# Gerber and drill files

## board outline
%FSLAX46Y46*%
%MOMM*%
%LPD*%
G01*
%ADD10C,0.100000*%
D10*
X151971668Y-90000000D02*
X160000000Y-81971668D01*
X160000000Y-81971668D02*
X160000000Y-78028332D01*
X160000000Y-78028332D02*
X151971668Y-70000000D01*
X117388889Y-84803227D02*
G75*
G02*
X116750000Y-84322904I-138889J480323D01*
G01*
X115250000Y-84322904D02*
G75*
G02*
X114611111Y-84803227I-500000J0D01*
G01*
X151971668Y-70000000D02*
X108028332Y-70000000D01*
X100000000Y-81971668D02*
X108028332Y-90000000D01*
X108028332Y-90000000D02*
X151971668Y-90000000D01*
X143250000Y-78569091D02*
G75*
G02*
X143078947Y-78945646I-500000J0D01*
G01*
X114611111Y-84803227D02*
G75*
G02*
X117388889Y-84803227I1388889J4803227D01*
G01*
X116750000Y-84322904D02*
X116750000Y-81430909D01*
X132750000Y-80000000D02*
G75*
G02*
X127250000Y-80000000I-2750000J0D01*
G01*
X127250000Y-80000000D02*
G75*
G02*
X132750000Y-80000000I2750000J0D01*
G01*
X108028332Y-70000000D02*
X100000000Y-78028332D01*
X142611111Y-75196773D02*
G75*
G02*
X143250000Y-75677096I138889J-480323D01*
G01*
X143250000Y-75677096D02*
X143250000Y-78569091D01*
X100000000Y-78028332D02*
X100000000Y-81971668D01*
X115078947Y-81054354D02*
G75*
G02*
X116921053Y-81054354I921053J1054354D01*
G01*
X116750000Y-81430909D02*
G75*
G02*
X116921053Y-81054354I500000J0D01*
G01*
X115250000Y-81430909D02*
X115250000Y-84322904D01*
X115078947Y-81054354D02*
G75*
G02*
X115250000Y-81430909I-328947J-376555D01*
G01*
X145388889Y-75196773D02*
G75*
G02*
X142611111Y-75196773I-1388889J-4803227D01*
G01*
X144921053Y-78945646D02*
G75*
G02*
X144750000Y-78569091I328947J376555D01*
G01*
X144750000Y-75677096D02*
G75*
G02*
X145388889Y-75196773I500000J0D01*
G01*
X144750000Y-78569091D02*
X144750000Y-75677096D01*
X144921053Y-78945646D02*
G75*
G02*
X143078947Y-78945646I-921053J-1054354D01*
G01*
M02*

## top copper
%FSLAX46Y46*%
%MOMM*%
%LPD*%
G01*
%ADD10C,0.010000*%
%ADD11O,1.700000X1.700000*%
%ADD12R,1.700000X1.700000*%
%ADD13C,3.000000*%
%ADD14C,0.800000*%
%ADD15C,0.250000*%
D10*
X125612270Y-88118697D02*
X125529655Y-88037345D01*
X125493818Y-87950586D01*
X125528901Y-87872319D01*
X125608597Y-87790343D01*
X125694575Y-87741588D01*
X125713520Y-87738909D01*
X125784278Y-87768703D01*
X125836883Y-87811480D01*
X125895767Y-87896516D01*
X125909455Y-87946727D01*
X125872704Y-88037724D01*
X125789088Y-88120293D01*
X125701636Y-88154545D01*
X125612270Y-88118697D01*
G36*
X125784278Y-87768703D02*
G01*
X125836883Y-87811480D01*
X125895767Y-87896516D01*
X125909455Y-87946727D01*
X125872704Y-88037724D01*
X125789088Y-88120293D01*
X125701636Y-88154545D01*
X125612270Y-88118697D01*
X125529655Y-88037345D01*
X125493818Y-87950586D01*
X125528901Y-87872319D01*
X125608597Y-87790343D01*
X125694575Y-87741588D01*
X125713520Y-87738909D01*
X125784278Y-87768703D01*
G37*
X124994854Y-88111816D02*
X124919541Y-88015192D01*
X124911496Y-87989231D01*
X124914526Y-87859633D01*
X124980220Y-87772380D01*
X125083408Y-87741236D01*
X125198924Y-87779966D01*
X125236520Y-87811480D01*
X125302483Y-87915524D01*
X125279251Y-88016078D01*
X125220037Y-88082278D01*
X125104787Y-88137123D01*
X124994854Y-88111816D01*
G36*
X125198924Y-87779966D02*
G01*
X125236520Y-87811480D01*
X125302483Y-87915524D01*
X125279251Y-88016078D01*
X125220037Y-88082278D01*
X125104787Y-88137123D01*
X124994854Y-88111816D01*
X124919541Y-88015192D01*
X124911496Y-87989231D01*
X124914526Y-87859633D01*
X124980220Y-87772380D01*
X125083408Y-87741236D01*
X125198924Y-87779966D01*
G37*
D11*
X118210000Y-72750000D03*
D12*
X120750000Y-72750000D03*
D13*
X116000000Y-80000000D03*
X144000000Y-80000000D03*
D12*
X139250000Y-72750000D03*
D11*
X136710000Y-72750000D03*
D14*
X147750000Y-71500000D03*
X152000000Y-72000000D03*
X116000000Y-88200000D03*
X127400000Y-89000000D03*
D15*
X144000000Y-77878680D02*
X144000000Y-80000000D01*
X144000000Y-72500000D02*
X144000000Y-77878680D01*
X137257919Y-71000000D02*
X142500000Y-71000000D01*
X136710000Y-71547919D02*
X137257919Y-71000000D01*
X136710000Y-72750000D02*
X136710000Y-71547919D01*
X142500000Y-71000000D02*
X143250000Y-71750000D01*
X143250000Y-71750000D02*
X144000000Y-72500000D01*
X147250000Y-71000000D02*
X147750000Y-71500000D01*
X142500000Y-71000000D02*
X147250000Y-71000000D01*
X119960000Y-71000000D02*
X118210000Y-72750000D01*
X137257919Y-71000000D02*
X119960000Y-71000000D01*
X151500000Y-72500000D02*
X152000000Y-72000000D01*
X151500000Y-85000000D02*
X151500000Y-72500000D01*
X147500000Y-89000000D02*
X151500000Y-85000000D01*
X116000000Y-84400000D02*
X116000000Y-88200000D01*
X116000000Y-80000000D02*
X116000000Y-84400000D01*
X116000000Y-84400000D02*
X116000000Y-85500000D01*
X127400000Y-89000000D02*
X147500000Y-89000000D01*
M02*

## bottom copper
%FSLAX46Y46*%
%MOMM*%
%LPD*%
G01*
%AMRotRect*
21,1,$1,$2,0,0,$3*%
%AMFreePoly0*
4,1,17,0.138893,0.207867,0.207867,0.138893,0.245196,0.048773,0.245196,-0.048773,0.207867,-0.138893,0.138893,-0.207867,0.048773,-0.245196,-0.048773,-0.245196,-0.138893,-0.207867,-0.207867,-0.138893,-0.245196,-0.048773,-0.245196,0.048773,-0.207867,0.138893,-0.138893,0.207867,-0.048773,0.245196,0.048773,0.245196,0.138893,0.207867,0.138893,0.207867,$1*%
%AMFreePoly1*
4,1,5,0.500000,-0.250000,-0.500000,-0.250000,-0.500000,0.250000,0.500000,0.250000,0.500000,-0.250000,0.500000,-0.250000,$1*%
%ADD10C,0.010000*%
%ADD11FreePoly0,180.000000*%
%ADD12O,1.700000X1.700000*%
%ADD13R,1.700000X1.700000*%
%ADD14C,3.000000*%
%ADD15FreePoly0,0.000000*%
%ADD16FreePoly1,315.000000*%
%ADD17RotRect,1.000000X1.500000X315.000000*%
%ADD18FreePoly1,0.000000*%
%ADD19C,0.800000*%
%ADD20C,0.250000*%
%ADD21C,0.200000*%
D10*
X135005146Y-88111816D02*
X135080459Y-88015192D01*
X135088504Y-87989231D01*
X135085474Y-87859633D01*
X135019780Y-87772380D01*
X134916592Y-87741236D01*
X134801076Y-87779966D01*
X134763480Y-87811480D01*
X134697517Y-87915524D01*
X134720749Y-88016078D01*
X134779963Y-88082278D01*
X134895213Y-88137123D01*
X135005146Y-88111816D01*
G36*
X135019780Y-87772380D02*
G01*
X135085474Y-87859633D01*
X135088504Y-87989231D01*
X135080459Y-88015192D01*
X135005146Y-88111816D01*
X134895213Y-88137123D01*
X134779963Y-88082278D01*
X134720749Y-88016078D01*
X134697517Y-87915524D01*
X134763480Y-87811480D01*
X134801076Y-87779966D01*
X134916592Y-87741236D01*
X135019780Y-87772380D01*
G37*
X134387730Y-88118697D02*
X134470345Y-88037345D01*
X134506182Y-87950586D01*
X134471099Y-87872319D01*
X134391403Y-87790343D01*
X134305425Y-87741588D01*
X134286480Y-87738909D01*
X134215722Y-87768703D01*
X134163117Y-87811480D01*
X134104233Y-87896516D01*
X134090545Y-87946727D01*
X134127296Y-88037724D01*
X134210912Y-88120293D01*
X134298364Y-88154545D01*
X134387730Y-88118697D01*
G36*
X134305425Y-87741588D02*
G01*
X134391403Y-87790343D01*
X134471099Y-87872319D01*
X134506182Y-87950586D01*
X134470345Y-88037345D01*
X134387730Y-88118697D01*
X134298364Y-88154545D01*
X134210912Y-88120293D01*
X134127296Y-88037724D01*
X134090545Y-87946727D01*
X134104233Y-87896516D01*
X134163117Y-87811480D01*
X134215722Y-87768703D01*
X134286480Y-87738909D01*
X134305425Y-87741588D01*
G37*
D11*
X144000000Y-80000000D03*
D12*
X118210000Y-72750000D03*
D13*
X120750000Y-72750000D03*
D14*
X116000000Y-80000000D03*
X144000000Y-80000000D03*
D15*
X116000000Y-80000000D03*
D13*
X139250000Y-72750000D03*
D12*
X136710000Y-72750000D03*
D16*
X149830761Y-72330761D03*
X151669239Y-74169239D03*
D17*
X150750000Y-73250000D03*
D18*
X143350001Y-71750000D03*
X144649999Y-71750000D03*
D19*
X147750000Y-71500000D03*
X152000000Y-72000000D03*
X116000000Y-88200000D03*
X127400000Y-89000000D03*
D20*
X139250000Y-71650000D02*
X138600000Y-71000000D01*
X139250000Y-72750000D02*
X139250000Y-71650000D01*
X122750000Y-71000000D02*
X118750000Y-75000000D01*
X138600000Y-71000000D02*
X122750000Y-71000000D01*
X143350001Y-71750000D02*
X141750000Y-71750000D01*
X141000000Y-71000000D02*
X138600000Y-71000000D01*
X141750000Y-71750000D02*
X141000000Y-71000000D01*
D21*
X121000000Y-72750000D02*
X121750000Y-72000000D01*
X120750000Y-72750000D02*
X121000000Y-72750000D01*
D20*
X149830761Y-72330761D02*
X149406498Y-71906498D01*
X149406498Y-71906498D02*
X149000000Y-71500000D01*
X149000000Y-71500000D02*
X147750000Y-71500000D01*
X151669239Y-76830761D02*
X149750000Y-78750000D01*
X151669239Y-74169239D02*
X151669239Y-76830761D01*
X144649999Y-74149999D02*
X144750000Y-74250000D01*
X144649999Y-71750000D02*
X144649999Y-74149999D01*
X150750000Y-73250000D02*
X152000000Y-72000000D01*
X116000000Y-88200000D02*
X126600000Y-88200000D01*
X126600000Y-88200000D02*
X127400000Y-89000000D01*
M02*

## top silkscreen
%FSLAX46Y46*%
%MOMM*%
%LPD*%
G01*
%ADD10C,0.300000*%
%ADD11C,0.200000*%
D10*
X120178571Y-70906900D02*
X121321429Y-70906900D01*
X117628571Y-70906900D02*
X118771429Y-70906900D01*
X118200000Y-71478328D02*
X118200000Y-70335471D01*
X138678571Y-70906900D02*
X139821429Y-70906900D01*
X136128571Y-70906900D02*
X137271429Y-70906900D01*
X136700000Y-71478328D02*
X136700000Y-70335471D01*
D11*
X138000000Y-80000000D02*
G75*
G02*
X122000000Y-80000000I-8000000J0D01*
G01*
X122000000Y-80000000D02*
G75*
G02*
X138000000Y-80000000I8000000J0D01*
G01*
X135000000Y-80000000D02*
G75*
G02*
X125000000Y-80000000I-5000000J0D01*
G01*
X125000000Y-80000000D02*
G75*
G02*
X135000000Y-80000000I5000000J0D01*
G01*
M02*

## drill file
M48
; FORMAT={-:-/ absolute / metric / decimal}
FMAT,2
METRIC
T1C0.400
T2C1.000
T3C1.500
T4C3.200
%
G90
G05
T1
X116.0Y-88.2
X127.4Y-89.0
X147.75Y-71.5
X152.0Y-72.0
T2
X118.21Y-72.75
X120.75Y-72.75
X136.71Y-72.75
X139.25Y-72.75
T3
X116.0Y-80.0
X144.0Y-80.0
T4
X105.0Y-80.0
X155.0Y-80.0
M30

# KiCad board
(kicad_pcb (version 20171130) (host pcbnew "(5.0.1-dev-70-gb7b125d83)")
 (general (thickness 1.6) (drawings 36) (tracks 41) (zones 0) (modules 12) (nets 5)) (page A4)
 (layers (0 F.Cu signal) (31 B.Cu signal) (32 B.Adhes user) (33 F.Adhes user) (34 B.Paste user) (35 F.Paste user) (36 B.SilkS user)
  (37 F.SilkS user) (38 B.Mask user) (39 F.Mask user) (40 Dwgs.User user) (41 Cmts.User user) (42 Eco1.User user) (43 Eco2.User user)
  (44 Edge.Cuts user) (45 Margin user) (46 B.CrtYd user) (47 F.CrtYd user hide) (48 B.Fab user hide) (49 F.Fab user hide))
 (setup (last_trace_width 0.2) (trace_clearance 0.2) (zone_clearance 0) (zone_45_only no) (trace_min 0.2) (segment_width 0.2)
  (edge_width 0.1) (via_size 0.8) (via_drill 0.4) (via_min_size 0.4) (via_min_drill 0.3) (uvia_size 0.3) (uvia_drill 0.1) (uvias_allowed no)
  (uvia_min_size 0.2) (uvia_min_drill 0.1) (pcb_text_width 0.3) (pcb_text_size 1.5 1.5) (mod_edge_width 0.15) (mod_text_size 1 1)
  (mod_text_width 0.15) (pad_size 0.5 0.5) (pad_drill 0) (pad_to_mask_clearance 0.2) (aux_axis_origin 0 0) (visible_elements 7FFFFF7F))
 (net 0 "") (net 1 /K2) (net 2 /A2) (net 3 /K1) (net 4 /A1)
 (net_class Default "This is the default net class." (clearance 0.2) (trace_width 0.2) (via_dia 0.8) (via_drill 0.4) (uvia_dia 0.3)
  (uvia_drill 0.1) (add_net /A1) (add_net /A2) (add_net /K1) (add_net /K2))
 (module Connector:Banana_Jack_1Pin (layer F.Cu) (at 75.6 77.6 180)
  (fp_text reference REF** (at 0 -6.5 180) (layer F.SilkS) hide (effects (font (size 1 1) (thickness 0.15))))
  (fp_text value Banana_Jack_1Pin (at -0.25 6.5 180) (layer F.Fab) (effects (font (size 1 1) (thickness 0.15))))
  (pad e smd custom (at -68.4 -2.4 180) (size 0.5 0.5) (layers B.Cu B.Paste B.Mask) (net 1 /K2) (zone_connect 0)
   (options (clearance outline) (anchor circle)) (primitives)))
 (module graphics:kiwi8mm (layer F.Cu) (at 123 87 180)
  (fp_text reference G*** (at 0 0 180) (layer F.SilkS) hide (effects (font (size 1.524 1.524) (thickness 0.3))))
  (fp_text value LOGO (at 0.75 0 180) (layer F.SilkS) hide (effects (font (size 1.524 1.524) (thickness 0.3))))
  (fp_poly
   (pts (xy -2.61227 -1.118697) (xy -2.529655 -1.037345) (xy -2.493818 -0.950586) (xy -2.528901 -0.872319) (xy -2.608597 -0.790343)
    (xy -2.694575 -0.741588) (xy -2.71352 -0.738909) (xy -2.784278 -0.768703) (xy -2.836883 -0.81148) (xy -2.895767 -0.896516)
    (xy -2.909455 -0.946727) (xy -2.872704 -1.037724) (xy -2.789088 -1.120293) (xy -2.701636 -1.154545) (xy -2.61227 -1.118697))
   (layer F.Cu) (width 0.01))
  (fp_poly
   (pts (xy -1.994854 -1.111816) (xy -1.919541 -1.015192) (xy -1.911496 -0.989231) (xy -1.914526 -0.859633) (xy -1.98022 -0.77238)
    (xy -2.083408 -0.741236) (xy -2.198924 -0.779966) (xy -2.23652 -0.81148) (xy -2.302483 -0.915524) (xy -2.279251 -1.016078)
    (xy -2.220037 -1.082278) (xy -2.104787 -1.137123) (xy -1.994854 -1.111816))
   (layer F.Cu) (width 0.01)))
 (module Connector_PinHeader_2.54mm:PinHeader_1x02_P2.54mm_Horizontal (layer B.Cu) (at 120.75 72.75 90)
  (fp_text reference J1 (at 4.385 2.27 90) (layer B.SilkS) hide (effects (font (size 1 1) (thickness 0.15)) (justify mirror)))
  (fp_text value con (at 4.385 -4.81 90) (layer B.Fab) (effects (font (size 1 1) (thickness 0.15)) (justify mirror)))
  (pad 2 thru_hole oval (at 0 -2.54 90) (size 1.7 1.7) (drill 1) (layers *.Cu *.Mask) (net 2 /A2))
  (pad 1 thru_hole rect (at 0 0 90) (size 1.7 1.7) (drill 1) (layers *.Cu *.Mask) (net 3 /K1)))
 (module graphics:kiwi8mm (layer B.Cu) (at 137 87)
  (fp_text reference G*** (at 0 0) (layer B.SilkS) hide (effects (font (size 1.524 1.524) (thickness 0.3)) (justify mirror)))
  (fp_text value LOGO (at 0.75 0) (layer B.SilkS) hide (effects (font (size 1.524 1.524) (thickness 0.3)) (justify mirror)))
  (fp_poly
   (pts (xy -1.994854 1.111816) (xy -1.919541 1.015192) (xy -1.911496 0.989231) (xy -1.914526 0.859633) (xy -1.98022 0.77238)
    (xy -2.083408 0.741236) (xy -2.198924 0.779966) (xy -2.23652 0.81148) (xy -2.302483 0.915524) (xy -2.279251 1.016078)
    (xy -2.220037 1.082278) (xy -2.104787 1.137123) (xy -1.994854 1.111816))
   (layer B.Cu) (width 0.01))
  (fp_poly
   (pts (xy -2.61227 1.118697) (xy -2.529655 1.037345) (xy -2.493818 0.950586) (xy -2.528901 0.872319) (xy -2.608597 0.790343)
    (xy -2.694575 0.741588) (xy -2.71352 0.738909) (xy -2.784278 0.768703) (xy -2.836883 0.81148) (xy -2.895767 0.896516)
    (xy -2.909455 0.946727) (xy -2.872704 1.037724) (xy -2.789088 1.120293) (xy -2.701636 1.154545) (xy -2.61227 1.118697))
   (layer B.Cu) (width 0.01)))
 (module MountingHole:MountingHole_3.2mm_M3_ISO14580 (layer F.Cu) (at 105 80)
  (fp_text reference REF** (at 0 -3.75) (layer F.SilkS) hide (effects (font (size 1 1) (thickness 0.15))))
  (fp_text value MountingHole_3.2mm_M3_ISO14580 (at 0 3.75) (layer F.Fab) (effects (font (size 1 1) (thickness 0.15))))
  (pad 1 np_thru_hole circle (at 0 0) (size 3.2 3.2) (drill 3.2) (layers *.Cu *.Mask)))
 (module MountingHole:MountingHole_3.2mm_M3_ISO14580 (layer F.Cu) (at 155 80)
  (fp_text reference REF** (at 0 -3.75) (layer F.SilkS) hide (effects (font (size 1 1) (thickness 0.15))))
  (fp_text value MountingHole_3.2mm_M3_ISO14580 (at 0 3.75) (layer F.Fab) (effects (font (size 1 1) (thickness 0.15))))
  (pad 1 np_thru_hole circle (at 0 0) (size 3.2 3.2) (drill 3.2) (layers *.Cu *.Mask)))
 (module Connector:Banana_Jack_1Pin (layer F.Cu) (at 175.6 64.6)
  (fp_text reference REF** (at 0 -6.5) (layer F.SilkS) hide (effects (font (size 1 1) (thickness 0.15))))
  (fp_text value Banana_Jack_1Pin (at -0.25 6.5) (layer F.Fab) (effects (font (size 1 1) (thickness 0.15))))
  (pad 1 thru_hole circle (at -59.6 15.4) (size 3 3) (drill 1.5) (layers *.Cu *.Mask) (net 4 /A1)))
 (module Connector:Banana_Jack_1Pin (layer F.Cu) (at 203.6 64.6)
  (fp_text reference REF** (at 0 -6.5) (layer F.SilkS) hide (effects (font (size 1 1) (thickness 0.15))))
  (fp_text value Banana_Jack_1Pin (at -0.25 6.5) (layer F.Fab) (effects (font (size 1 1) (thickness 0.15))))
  (pad 1 thru_hole circle (at -59.6 15.4) (size 3 3) (drill 1.5) (layers *.Cu *.Mask) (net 2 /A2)))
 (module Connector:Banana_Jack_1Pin (layer F.Cu) (at 184.4 82.4)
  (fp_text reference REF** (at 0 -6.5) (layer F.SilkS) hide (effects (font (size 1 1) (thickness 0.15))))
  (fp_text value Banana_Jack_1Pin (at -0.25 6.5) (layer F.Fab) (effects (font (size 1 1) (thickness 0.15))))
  (pad e smd custom (at -68.4 -2.4) (size 0.5 0.5) (layers B.Cu B.Paste B.Mask) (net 3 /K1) (zone_connect 0)
   (options (clearance outline) (anchor circle)) (primitives)))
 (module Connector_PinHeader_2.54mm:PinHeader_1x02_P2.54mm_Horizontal (layer B.Cu) (at 139.25 72.75 90)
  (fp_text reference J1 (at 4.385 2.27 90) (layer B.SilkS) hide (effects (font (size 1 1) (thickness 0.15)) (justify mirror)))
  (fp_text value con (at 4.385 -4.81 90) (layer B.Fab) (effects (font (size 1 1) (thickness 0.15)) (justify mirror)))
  (pad 1 thru_hole rect (at 0 0 90) (size 1.7 1.7) (drill 1) (layers *.Cu *.Mask) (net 3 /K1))
  (pad 2 thru_hole oval (at 0 -2.54 90) (size 1.7 1.7) (drill 1) (layers *.Cu *.Mask) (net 2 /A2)))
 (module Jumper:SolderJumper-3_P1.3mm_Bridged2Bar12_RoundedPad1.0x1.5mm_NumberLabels (layer B.Cu) (at 150.75 73.25 315)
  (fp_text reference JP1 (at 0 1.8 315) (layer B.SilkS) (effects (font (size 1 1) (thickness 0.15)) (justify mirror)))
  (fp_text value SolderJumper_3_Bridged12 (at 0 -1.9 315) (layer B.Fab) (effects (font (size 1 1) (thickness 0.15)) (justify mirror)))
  (pad 1 smd custom (at -1.3 0 315) (size 1 0.5) (layers B.Cu B.Mask) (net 2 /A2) (zone_connect 0)
   (options (clearance outline) (anchor rect)) (primitives))
  (pad 3 smd custom (at 1.3 0 315) (size 1 0.5) (layers B.Cu B.Mask) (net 1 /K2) (zone_connect 0)
   (options (clearance outline) (anchor rect)) (primitives))
  (pad 2 smd rect (at 0 0 315) (size 1 1.5) (layers B.Cu B.Mask) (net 4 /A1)))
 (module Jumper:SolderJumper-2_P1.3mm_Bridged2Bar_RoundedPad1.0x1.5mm (layer B.Cu) (at 144 71.75)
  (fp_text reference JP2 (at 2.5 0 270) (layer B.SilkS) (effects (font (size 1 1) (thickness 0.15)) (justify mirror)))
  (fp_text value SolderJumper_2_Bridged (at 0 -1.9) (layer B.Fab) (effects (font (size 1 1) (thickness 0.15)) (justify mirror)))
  (pad 1 smd custom (at -0.649999 0) (size 1 0.5) (layers B.Cu B.Mask) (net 3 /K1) (zone_connect 0)
   (options (clearance outline) (anchor rect)) (primitives))
  (pad 2 smd custom (at 0.649999 0) (size 1 0.5) (layers B.Cu B.Mask) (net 1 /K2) (zone_connect 0)
   (options (clearance outline) (anchor rect)) (primitives)))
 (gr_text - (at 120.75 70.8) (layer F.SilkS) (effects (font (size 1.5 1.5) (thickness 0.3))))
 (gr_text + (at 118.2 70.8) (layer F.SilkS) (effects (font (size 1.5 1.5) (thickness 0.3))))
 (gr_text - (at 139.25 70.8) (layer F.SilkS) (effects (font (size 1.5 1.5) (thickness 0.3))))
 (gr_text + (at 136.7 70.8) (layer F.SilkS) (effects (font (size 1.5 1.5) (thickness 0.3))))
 (gr_line (start 151.971668 90) (end 160 81.971668) (layer Edge.Cuts) (width 0.1))
 (gr_line (start 160 81.971668) (end 160 78.028332) (layer Edge.Cuts) (width 0.1))
 (gr_line (start 160 78.028332) (end 151.971668 70) (layer Edge.Cuts) (width 0.1))
 (gr_circle (center 130 80) (end 138 80) (layer F.SilkS) (width 0.2))
 (gr_circle (center 130 80) (end 125 80) (layer F.SilkS) (width 0.2))
 (gr_arc (start 117.25 84.322904) (end 116.75 84.322904) (angle -106.1276202) (layer Edge.Cuts) (width 0.1))
 (gr_arc (start 114.75 84.322904) (end 114.611111 84.803227) (angle -106.1276202) (layer Edge.Cuts) (width 0.1))
 (gr_line (start 151.971668 70) (end 108.028332 70) (layer Edge.Cuts) (width 0.1))
 (gr_line (start 100 81.971668) (end 108.028332 90) (layer Edge.Cuts) (width 0.1))
 (gr_line (start 108.028332 90) (end 151.971668 90) (layer Edge.Cuts) (width 0.1))
 (gr_arc (start 142.75 78.569091) (end 143.078947 78.945646) (angle -48.86048959) (layer Edge.Cuts) (width 0.1))
 (gr_arc (start 116 80) (end 117.388889 84.803227) (angle -327.7447596) (layer Edge.Cuts) (width 0.1))
 (gr_line (start 116.75 84.322904) (end 116.75 81.430909) (layer Edge.Cuts) (width 0.1))
 (gr_circle (center 130 80) (end 132.75 80) (layer Edge.Cuts) (width 0.1))
 (gr_line (start 108.028332 70) (end 100 78.028332) (layer Edge.Cuts) (width 0.1))
 (gr_arc (start 142.75 75.677096) (end 143.25 75.677096) (angle -106.1276202) (layer Edge.Cuts) (width 0.1))
 (gr_line (start 143.25 75.677096) (end 143.25 78.569091) (layer Edge.Cuts) (width 0.1))
 (gr_line (start 100 78.028332) (end 100 81.971668) (layer Edge.Cuts) (width 0.1))
 (gr_arc (start 116 80) (end 116.921053 81.054354) (angle -277.7209792) (layer Edge.Cuts) (width 0.1))
 (gr_arc (start 117.25 81.430909) (end 116.921053 81.054354) (angle -48.86048959) (layer Edge.Cuts) (width 0.1))
 (gr_line (start 115.25 81.430909) (end 115.25 84.322904) (layer Edge.Cuts) (width 0.1))
 (gr_arc (start 114.75 81.430909) (end 115.25 81.430909) (angle -48.86048959) (layer Edge.Cuts) (width 0.1))
 (gr_arc (start 144 80) (end 142.611111 75.196773) (angle -327.7447596) (layer Edge.Cuts) (width 0.1))
 (gr_arc (start 145.25 78.569091) (end 144.75 78.569091) (angle -48.86048959) (layer Edge.Cuts) (width 0.1))
 (gr_arc (start 145.25 75.677096) (end 145.388889 75.196773) (angle -106.1276202) (layer Edge.Cuts) (width 0.1))
 (gr_line (start 144.75 78.569091) (end 144.75 75.677096) (layer Edge.Cuts) (width 0.1))
 (gr_arc (start 144 80) (end 143.078947 78.945646) (angle -277.7209792) (layer Edge.Cuts) (width 0.1))
 (segment (start 139.25 71.65) (end 138.6 71) (width 0.25) (layer B.Cu) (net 3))
 (segment (start 139.25 72.75) (end 139.25 71.65) (width 0.25) (layer B.Cu) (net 3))
 (segment (start 122.75 71) (end 118.75 75) (width 0.25) (layer B.Cu) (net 3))
 (segment (start 138.6 71) (end 122.75 71) (width 0.25) (layer B.Cu) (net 3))
 (segment (start 143.350001 71.75) (end 141.75 71.75) (width 0.25) (layer B.Cu) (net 3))
 (segment (start 141 71) (end 138.6 71) (width 0.25) (layer B.Cu) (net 3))
 (segment (start 141.75 71.75) (end 141 71) (width 0.25) (layer B.Cu) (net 3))
 (segment (start 121 72.75) (end 121.75 72) (width 0.2) (layer B.Cu) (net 3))
 (segment (start 120.75 72.75) (end 121 72.75) (width 0.2) (layer B.Cu) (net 3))
 (segment (start 144 77.87868) (end 144 80) (width 0.25) (layer F.Cu) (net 2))
 (segment (start 144 72.5) (end 144 77.87868) (width 0.25) (layer F.Cu) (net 2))
 (segment (start 137.257919 71) (end 142.5 71) (width 0.25) (layer F.Cu) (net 2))
 (segment (start 136.71 71.547919) (end 137.257919 71) (width 0.25) (layer F.Cu) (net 2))
 (segment (start 136.71 72.75) (end 136.71 71.547919) (width 0.25) (layer F.Cu) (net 2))
 (segment (start 142.5 71) (end 143.25 71.75) (width 0.25) (layer F.Cu) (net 2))
 (segment (start 143.25 71.75) (end 144 72.5) (width 0.25) (layer F.Cu) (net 2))
 (segment (start 149.830761 72.330761) (end 149.406498 71.906498) (width 0.25) (layer B.Cu) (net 2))
 (segment (start 149.406498 71.906498) (end 149 71.5) (width 0.25) (layer B.Cu) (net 2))
 (via (at 147.75 71.5) (size 0.8) (drill 0.4) (layers F.Cu B.Cu) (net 2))
 (segment (start 149 71.5) (end 147.75 71.5) (width 0.25) (layer B.Cu) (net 2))
 (segment (start 147.25 71) (end 147.75 71.5) (width 0.25) (layer F.Cu) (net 2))
 (segment (start 142.5 71) (end 147.25 71) (width 0.25) (layer F.Cu) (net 2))
 (segment (start 119.96 71) (end 118.21 72.75) (width 0.25) (layer F.Cu) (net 2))
 (segment (start 137.257919 71) (end 119.96 71) (width 0.25) (layer F.Cu) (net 2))
 (segment (start 151.669239 76.830761) (end 149.75 78.75) (width 0.25) (layer B.Cu) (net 1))
 (segment (start 151.669239 74.169239) (end 151.669239 76.830761) (width 0.25) (layer B.Cu) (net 1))
 (segment (start 144.649999 74.149999) (end 144.75 74.25) (width 0.25) (layer B.Cu) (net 1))
 (segment (start 144.649999 71.75) (end 144.649999 74.149999) (width 0.25) (layer B.Cu) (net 1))
 (via (at 152 72) (size 0.8) (drill 0.4) (layers F.Cu B.Cu) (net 4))
 (segment (start 150.75 73.25) (end 152 72) (width 0.25) (layer B.Cu) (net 4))
 (segment (start 151.5 72.5) (end 152 72) (width 0.25) (layer F.Cu) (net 4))
 (segment (start 151.5 85) (end 151.5 72.5) (width 0.25) (layer F.Cu) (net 4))
 (segment (start 147.5 89) (end 151.5 85) (width 0.25) (layer F.Cu) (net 4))
 (via (at 116 88.2) (size 0.8) (drill 0.4) (layers F.Cu B.Cu) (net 4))
 (segment (start 116 84.4) (end 116 88.2) (width 0.25) (layer F.Cu) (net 4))
 (segment (start 116 80) (end 116 84.4) (width 0.25) (layer F.Cu) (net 4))
 (segment (start 116 84.4) (end 116 85.5) (width 0.25) (layer F.Cu) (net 4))
 (via (at 127.4 89) (size 0.8) (drill 0.4) (layers F.Cu B.Cu) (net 4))
 (segment (start 116 88.2) (end 126.6 88.2) (width 0.25) (layer B.Cu) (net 4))
 (segment (start 126.6 88.2) (end 127.4 89) (width 0.25) (layer B.Cu) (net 4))
 (segment (start 127.4 89) (end 147.5 89) (width 0.25) (layer F.Cu) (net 4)))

